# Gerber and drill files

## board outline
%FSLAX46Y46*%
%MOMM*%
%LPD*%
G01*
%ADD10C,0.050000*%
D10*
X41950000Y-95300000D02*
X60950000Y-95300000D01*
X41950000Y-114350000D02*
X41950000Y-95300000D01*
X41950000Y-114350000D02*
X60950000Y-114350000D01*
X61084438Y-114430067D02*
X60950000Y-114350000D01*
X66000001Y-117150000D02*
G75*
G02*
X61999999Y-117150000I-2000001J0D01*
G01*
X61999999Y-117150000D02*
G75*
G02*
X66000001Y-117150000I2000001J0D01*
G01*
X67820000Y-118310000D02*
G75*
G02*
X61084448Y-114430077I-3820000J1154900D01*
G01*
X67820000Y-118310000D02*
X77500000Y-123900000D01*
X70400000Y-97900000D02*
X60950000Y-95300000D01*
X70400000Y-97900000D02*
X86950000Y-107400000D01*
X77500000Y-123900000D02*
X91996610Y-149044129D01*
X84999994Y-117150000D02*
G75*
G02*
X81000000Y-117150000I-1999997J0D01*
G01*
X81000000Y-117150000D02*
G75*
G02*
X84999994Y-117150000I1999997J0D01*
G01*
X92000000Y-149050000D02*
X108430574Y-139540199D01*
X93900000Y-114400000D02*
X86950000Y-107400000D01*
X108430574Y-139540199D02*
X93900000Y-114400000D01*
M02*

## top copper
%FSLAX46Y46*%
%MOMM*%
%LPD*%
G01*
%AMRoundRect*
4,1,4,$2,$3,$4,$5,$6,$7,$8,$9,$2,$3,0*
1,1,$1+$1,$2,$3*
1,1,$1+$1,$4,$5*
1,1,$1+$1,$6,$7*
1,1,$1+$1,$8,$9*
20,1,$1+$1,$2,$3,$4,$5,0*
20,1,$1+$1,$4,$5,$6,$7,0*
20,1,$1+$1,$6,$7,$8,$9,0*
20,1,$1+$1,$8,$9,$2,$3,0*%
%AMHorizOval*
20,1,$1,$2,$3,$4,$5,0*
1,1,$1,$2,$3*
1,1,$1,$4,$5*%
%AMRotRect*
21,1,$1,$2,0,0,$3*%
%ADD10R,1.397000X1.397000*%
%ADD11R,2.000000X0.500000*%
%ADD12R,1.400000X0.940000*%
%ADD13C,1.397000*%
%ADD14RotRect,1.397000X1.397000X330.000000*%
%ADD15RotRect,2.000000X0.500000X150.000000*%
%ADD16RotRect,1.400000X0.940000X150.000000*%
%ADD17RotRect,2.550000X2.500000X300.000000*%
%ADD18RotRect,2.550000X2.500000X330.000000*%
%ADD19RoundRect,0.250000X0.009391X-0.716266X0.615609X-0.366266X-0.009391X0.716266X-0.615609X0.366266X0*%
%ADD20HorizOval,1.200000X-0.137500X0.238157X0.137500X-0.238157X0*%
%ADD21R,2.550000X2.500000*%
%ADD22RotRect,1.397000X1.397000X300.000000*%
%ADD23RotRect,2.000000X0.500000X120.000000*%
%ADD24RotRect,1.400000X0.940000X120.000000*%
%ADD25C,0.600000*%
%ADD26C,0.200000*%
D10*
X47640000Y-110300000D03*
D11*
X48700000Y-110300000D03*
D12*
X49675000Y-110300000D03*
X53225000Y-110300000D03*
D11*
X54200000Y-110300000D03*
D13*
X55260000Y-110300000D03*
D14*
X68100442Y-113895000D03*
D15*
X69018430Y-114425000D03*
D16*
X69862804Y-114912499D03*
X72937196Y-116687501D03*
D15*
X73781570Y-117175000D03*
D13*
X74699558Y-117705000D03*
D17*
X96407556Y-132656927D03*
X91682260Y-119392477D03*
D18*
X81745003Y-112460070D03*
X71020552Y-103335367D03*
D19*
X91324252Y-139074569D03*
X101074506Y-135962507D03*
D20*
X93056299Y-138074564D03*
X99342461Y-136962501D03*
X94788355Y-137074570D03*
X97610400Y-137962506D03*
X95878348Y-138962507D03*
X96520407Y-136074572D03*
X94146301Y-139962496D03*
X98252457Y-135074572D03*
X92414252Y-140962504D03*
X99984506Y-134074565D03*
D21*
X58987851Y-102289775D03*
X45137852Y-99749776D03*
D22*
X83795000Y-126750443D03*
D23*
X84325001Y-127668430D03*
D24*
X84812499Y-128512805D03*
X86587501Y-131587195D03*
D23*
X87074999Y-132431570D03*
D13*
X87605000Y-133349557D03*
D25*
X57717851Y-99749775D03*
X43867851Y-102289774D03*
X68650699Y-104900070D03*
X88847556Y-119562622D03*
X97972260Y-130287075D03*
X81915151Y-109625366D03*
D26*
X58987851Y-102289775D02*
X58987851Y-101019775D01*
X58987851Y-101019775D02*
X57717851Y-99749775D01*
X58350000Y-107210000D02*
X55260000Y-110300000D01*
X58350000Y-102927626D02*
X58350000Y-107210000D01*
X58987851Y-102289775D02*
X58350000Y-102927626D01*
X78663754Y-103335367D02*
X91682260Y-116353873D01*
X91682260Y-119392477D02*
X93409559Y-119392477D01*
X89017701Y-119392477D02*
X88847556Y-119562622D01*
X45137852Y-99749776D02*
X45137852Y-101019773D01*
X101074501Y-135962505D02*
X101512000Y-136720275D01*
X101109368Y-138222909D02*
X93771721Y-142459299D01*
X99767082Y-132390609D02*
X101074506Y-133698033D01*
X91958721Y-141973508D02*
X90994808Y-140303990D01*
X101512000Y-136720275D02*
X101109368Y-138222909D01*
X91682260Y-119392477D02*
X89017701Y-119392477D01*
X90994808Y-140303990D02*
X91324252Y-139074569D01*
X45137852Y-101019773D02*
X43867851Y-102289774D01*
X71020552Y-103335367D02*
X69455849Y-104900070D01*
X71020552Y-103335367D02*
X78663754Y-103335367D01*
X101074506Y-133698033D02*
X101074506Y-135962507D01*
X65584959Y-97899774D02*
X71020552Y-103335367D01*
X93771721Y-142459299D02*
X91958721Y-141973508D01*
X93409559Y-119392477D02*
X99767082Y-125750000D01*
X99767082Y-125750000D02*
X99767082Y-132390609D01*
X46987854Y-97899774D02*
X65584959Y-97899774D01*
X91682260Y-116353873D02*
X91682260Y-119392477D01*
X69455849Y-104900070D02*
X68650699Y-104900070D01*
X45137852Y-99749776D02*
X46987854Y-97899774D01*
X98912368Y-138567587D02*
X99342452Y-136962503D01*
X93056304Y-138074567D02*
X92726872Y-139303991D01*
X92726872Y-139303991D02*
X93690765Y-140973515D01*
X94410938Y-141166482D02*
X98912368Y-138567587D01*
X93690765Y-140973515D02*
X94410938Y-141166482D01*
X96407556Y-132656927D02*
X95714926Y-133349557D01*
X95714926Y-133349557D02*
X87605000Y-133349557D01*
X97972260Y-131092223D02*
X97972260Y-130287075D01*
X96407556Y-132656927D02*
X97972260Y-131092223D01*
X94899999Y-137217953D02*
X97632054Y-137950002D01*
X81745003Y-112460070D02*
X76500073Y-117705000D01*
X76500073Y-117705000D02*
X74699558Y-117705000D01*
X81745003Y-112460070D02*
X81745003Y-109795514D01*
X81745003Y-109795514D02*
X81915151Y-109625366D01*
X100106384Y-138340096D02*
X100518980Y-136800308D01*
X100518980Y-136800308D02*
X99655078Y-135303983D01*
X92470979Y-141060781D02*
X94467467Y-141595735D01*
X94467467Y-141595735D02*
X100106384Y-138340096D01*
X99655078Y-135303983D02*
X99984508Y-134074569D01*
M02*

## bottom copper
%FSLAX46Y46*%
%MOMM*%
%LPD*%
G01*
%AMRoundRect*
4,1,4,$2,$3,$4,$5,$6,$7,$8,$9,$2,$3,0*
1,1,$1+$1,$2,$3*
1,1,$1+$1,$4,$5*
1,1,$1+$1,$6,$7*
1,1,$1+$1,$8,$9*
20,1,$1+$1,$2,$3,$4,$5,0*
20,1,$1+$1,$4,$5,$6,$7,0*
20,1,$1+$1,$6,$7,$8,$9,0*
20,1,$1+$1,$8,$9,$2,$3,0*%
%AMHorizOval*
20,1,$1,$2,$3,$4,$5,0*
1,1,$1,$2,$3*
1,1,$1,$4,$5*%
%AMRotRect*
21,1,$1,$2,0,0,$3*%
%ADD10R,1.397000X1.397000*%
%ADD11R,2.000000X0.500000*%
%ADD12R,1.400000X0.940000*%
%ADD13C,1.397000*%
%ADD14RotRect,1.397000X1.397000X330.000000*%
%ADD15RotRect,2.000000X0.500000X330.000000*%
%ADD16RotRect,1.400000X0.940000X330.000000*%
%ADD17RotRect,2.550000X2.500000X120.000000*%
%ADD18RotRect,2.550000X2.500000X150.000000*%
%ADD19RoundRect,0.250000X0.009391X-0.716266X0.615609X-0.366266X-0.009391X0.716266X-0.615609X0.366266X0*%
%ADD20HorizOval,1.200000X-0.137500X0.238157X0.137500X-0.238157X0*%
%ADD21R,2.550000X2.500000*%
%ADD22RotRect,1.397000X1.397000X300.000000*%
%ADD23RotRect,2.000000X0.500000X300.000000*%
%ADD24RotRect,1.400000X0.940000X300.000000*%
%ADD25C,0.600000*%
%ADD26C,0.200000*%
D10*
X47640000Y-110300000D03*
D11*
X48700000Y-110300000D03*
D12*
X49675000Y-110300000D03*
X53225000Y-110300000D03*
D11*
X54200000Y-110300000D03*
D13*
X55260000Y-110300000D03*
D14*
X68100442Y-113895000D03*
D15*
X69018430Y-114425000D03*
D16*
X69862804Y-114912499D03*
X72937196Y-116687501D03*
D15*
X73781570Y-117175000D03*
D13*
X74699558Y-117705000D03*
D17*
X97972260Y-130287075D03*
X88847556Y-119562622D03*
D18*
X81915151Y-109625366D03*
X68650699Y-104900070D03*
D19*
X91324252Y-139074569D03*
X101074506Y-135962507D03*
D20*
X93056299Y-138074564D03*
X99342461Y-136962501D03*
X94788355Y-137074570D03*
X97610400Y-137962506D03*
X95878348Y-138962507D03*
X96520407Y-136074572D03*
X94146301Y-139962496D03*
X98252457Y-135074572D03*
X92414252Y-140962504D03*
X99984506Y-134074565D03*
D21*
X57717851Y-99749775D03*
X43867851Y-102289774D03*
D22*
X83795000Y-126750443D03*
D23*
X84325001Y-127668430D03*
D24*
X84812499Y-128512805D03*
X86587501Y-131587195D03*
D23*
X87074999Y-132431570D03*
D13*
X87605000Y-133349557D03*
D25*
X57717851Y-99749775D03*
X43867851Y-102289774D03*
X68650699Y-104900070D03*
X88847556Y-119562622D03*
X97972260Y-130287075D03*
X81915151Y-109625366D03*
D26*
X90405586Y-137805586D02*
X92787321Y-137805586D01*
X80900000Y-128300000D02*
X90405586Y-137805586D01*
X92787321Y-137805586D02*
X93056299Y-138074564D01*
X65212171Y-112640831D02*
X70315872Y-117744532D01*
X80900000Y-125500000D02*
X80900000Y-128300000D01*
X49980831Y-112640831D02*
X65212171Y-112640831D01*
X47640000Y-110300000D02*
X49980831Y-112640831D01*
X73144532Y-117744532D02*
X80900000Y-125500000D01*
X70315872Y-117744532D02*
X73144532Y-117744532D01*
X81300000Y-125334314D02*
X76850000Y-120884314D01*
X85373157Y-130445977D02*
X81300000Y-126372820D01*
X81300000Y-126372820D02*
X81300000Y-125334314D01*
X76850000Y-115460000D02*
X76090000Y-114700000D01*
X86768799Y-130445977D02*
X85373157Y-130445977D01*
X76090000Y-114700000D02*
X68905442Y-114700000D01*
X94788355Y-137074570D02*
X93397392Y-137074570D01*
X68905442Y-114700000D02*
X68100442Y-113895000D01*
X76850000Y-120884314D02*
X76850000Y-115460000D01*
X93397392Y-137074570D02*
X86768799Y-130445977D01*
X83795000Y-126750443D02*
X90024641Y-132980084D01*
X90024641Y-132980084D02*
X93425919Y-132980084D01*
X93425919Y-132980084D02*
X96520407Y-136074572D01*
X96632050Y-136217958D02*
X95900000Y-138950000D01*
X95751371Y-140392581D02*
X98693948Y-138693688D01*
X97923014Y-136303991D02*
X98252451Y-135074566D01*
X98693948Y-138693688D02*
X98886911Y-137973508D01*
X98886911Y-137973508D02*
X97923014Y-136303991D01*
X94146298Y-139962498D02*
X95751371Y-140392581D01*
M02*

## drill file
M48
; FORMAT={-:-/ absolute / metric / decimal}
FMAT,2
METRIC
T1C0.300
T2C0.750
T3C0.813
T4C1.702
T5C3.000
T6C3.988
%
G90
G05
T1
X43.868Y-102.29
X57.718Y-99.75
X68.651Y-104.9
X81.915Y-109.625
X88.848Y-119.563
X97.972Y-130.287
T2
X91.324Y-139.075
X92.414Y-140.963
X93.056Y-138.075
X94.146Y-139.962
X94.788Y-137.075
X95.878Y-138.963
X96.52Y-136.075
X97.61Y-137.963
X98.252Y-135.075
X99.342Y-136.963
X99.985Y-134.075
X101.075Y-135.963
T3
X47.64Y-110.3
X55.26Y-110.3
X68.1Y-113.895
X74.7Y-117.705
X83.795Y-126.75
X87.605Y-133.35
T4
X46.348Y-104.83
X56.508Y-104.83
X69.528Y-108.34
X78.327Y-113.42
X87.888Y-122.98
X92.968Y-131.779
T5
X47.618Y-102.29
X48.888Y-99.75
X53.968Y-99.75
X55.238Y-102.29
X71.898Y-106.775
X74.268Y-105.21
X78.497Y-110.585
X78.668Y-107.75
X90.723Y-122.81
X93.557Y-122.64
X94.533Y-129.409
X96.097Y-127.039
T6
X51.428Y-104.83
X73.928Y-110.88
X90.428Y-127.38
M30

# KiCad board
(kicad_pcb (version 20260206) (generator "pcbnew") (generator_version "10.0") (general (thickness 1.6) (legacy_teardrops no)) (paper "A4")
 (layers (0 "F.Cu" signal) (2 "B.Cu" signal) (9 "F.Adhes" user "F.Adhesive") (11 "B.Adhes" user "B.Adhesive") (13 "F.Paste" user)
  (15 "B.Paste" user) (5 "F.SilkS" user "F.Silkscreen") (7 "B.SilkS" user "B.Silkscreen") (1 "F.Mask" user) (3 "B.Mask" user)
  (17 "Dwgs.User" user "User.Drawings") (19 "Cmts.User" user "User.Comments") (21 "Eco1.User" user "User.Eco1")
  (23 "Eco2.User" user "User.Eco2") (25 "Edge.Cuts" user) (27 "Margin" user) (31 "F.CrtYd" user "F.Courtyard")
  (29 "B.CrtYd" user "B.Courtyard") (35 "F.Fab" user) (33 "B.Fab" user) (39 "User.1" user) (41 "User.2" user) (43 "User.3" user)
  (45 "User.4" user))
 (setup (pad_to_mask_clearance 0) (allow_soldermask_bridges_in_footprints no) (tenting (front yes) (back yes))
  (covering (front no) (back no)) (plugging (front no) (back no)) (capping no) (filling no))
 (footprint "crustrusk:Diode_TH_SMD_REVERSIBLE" (layer "F.Cu") (at 51.45 110.3)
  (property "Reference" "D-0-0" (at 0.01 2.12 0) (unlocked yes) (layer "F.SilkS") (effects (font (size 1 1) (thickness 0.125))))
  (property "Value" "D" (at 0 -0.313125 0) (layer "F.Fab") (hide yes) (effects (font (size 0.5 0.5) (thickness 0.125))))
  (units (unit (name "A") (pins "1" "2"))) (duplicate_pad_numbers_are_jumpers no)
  (pad "1" thru_hole rect (at -3.81 0) (size 1.397 1.397) (drill 0.8128) (layers "*.Cu" "*.Mask") (remove_unused_layers no) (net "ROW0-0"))
  (pad "1" smd rect (at -2.75 0 180) (size 2 0.5) (layers "F.Cu") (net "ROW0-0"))
  (pad "1" smd rect (at -2.75 0) (size 2 0.5) (layers "B.Cu") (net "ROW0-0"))
  (pad "1" smd rect (at -1.775 0 180) (size 1.4 0.94) (layers "F.Cu" "F.Mask" "F.Paste") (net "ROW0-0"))
  (pad "1" smd rect (at -1.775 0) (size 1.4 0.94) (layers "B.Cu" "B.Mask" "B.Paste") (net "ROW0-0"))
  (pad "2" smd rect (at 1.775 0 180) (size 1.4 0.94) (layers "F.Cu" "F.Mask" "F.Paste") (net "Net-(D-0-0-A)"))
  (pad "2" smd rect (at 1.775 0) (size 1.4 0.94) (layers "B.Cu" "B.Mask" "B.Paste") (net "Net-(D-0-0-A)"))
  (pad "2" smd rect (at 2.75 0 180) (size 2 0.5) (layers "F.Cu") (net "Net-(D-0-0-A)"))
  (pad "2" smd rect (at 2.75 0) (size 2 0.5) (layers "B.Cu") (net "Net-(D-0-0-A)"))
  (pad "2" thru_hole circle (at 3.81 0) (size 1.397 1.397) (drill 0.8128) (layers "*.Cu" "*.Mask") (remove_unused_layers no)
   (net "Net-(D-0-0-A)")))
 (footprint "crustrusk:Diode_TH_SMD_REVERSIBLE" (layer "F.Cu") (at 71.4 115.8 -30)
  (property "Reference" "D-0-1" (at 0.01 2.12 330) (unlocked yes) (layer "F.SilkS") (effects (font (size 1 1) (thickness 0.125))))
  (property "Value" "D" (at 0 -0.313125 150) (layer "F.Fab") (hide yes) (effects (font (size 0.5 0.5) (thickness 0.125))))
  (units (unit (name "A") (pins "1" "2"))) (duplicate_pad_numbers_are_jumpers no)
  (pad "1" thru_hole rect (at -3.810001 0.000001 330) (size 1.397 1.397) (drill 0.8128) (layers "*.Cu" "*.Mask") (remove_unused_layers no)
   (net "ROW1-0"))
  (pad "1" smd rect (at -2.75 0 150) (size 2 0.5) (layers "F.Cu") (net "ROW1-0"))
  (pad "1" smd rect (at -2.75 0 330) (size 2 0.5) (layers "B.Cu") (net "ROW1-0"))
  (pad "1" smd rect (at -1.775001 0 150) (size 1.4 0.94) (layers "F.Cu" "F.Mask" "F.Paste") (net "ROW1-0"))
  (pad "1" smd rect (at -1.775001 0 330) (size 1.4 0.94) (layers "B.Cu" "B.Mask" "B.Paste") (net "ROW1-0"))
  (pad "2" smd rect (at 1.775001 0 150) (size 1.4 0.94) (layers "F.Cu" "F.Mask" "F.Paste") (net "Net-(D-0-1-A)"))
  (pad "2" smd rect (at 1.775001 0 330) (size 1.4 0.94) (layers "B.Cu" "B.Mask" "B.Paste") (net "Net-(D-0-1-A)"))
  (pad "2" smd rect (at 2.75 0 150) (size 2 0.5) (layers "F.Cu") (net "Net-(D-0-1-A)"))
  (pad "2" smd rect (at 2.75 0 330) (size 2 0.5) (layers "B.Cu") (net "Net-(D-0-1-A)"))
  (pad "2" thru_hole circle (at 3.810001 -0.000001 330) (size 1.397 1.397) (drill 0.8128) (layers "*.Cu" "*.Mask") (remove_unused_layers no)
   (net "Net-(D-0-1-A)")))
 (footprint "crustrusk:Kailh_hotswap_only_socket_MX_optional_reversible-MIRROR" (layer "F.Cu") (at 90.427851 127.379775 -60)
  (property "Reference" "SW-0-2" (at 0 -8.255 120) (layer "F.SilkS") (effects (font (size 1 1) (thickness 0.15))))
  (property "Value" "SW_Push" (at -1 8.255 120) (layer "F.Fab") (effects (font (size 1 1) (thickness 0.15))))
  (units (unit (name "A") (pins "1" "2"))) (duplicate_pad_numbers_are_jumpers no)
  (pad "" np_thru_hole circle (at -5.08 0 300) (size 1.7018 1.7018) (drill 1.7018) (layers "*.Cu" "*.Mask"))
  (pad "" np_thru_hole circle (at -3.81 -2.540001 120) (size 3 3) (drill 3) (layers "*.Cu" "*.Mask"))
  (pad "" np_thru_hole circle (at -2.540001 -5.079998 300) (size 3 3) (drill 3) (layers "*.Cu" "*.Mask"))
  (pad "" np_thru_hole circle (at 0 0 300) (size 3.9878 3.9878) (drill 3.9878) (layers "*.Cu" "*.Mask"))
  (pad "" np_thru_hole circle (at 2.540002 -5.080001 120) (size 3 3) (drill 3) (layers "*.Cu" "*.Mask"))
  (pad "" np_thru_hole circle (at 3.81 -2.54 300) (size 3 3) (drill 3) (layers "*.Cu" "*.Mask"))
  (pad "" np_thru_hole circle (at 5.08 0 300) (size 1.7018 1.7018) (drill 1.7018) (layers "*.Cu" "*.Mask"))
  (pad "1" smd rect (at 6.29 -5.08 120) (size 2.55 2.5) (layers "B.Cu" "B.Mask" "B.Paste") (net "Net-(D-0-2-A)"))
  (pad "1" smd rect (at 7.56 -2.54 300) (size 2.55 2.5) (layers "F.Cu" "F.Mask" "F.Paste") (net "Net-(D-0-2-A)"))
  (pad "2" smd rect (at -7.560001 -2.540001 120) (size 2.55 2.5) (layers "B.Cu" "B.Mask" "B.Paste") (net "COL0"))
  (pad "2" smd rect (at -6.289998 -5.079999 300) (size 2.55 2.5) (layers "F.Cu" "F.Mask" "F.Paste") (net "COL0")))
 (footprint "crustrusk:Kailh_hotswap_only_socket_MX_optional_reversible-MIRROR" (layer "F.Cu") (at 73.927851 110.879775 -30)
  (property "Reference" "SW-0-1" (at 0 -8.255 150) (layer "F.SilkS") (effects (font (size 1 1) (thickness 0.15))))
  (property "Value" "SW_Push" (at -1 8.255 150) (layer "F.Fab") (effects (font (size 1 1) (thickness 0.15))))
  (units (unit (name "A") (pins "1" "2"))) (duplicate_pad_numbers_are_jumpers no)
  (pad "" np_thru_hole circle (at -5.08 0 330) (size 1.7018 1.7018) (drill 1.7018) (layers "*.Cu" "*.Mask"))
  (pad "" np_thru_hole circle (at -3.81 -2.54 150) (size 3 3) (drill 3) (layers "*.Cu" "*.Mask"))
  (pad "" np_thru_hole circle (at -2.54 -5.079997 330) (size 3 3) (drill 3) (layers "*.Cu" "*.Mask"))
  (pad "" np_thru_hole circle (at 0 0 330) (size 3.9878 3.9878) (drill 3.9878) (layers "*.Cu" "*.Mask"))
  (pad "" np_thru_hole circle (at 2.540002 -5.080001 150) (size 3 3) (drill 3) (layers "*.Cu" "*.Mask"))
  (pad "" np_thru_hole circle (at 3.81 -2.540001 330) (size 3 3) (drill 3) (layers "*.Cu" "*.Mask"))
  (pad "" np_thru_hole circle (at 5.08 0 330) (size 1.7018 1.7018) (drill 1.7018) (layers "*.Cu" "*.Mask"))
  (pad "1" smd rect (at 6.29 -5.08 150) (size 2.55 2.5) (layers "B.Cu" "B.Mask" "B.Paste") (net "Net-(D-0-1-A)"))
  (pad "1" smd rect (at 7.56 -2.54 330) (size 2.55 2.5) (layers "F.Cu" "F.Mask" "F.Paste") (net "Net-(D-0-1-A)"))
  (pad "2" smd rect (at -7.56 -2.54 150) (size 2.55 2.5) (layers "B.Cu" "B.Mask" "B.Paste") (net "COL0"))
  (pad "2" smd rect (at -6.289999 -5.079999 330) (size 2.55 2.5) (layers "F.Cu" "F.Mask" "F.Paste") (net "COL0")))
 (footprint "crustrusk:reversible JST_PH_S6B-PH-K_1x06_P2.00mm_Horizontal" (layer "F.Cu") (at 91.324252 139.074569 30)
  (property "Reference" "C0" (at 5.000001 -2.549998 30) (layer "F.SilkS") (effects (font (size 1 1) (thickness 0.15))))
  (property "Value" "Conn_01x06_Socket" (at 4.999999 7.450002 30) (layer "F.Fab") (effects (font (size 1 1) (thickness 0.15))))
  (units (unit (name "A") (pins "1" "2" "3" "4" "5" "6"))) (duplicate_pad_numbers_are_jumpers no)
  (pad "1" thru_hole roundrect (at 0 0 30) (size 1.2 1.75) (drill 0.75) (layers "*.Cu" "*.Mask") (remove_unused_layers no)
   (roundrect_rratio 0.208333) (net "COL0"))
  (pad "1" thru_hole roundrect (at 9.999999 2.180002 30) (size 1.2 1.75) (drill 0.75) (layers "*.Cu" "*.Mask") (remove_unused_layers no)
   (roundrect_rratio 0.208333) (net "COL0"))
  (pad "2" thru_hole oval (at 1.999999 -0.000006 30) (size 1.2 1.75) (drill 0.75) (layers "*.Cu" "*.Mask") (remove_unused_layers no)
   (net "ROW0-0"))
  (pad "2" thru_hole oval (at 8.000007 2.18 30) (size 1.2 1.75) (drill 0.75) (layers "*.Cu" "*.Mask") (remove_unused_layers no)
   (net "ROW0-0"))
  (pad "3" thru_hole oval (at 4.000001 0.000002 30) (size 1.2 1.75) (drill 0.75) (layers "*.Cu" "*.Mask") (remove_unused_layers no)
   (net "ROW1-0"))
  (pad "3" thru_hole oval (at 5.999995 2.179999 30) (size 1.2 1.75) (drill 0.75) (layers "*.Cu" "*.Mask") (remove_unused_layers no)
   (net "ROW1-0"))
  (pad "4" thru_hole oval (at 3.999994 2.179999 30) (size 1.2 1.75) (drill 0.75) (layers "*.Cu" "*.Mask") (remove_unused_layers no)
   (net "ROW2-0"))
  (pad "4" thru_hole oval (at 6.000001 0.000004 30) (size 1.2 1.75) (drill 0.75) (layers "*.Cu" "*.Mask") (remove_unused_layers no)
   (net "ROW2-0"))
  (pad "5" thru_hole oval (at 2.000003 2.179992 30) (size 1.2 1.75) (drill 0.75) (layers "*.Cu" "*.Mask") (remove_unused_layers no)
   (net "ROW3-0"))
  (pad "5" thru_hole oval (at 8 0.000003 30) (size 1.2 1.75) (drill 0.75) (layers "*.Cu" "*.Mask") (remove_unused_layers no) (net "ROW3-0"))
  (pad "6" thru_hole oval (at 0 2.18 30) (size 1.2 1.75) (drill 0.75) (layers "*.Cu" "*.Mask") (remove_unused_layers no) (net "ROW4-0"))
  (pad "6" thru_hole oval (at 10.000002 -0.000004 30) (size 1.2 1.75) (drill 0.75) (layers "*.Cu" "*.Mask") (remove_unused_layers no)
   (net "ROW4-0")))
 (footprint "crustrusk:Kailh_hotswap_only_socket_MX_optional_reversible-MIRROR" (layer "F.Cu") (at 51.427851 104.829775)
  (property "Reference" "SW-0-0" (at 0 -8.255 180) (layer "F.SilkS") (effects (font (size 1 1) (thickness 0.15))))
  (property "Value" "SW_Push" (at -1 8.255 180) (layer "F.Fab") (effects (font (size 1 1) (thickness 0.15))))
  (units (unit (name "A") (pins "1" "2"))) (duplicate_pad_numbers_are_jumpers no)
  (pad "" np_thru_hole circle (at -5.08 0) (size 1.7018 1.7018) (drill 1.7018) (layers "*.Cu" "*.Mask"))
  (pad "" np_thru_hole circle (at -3.81 -2.54 180) (size 3 3) (drill 3) (layers "*.Cu" "*.Mask"))
  (pad "" np_thru_hole circle (at -2.54 -5.079998) (size 3 3) (drill 3) (layers "*.Cu" "*.Mask"))
  (pad "" np_thru_hole circle (at 0 0) (size 3.9878 3.9878) (drill 3.9878) (layers "*.Cu" "*.Mask"))
  (pad "" np_thru_hole circle (at 2.540002 -5.080001 180) (size 3 3) (drill 3) (layers "*.Cu" "*.Mask"))
  (pad "" np_thru_hole circle (at 3.81 -2.54) (size 3 3) (drill 3) (layers "*.Cu" "*.Mask"))
  (pad "" np_thru_hole circle (at 5.08 0) (size 1.7018 1.7018) (drill 1.7018) (layers "*.Cu" "*.Mask"))
  (pad "1" smd rect (at 6.29 -5.08 180) (size 2.55 2.5) (layers "B.Cu" "B.Mask" "B.Paste") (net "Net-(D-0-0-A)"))
  (pad "1" smd rect (at 7.56 -2.54) (size 2.55 2.5) (layers "F.Cu" "F.Mask" "F.Paste") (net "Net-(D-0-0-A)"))
  (pad "2" smd rect (at -7.56 -2.540001 180) (size 2.55 2.5) (layers "B.Cu" "B.Mask" "B.Paste") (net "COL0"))
  (pad "2" smd rect (at -6.289999 -5.079999) (size 2.55 2.5) (layers "F.Cu" "F.Mask" "F.Paste") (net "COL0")))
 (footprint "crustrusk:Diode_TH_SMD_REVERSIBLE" (layer "F.Cu") (at 85.7 130.05 -60)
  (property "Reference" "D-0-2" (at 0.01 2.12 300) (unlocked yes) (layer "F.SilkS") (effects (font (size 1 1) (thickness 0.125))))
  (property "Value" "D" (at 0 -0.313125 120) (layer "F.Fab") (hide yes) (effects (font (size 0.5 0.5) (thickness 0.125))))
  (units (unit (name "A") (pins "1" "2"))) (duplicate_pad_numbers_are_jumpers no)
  (pad "1" thru_hole rect (at -3.81 0 300) (size 1.397 1.397) (drill 0.8128) (layers "*.Cu" "*.Mask") (remove_unused_layers no)
   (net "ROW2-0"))
  (pad "1" smd rect (at -2.75 -0.000001 120) (size 2 0.5) (layers "F.Cu") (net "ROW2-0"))
  (pad "1" smd rect (at -2.75 -0.000001 300) (size 2 0.5) (layers "B.Cu") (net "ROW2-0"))
  (pad "1" smd rect (at -1.775 0.000001 120) (size 1.4 0.94) (layers "F.Cu" "F.Mask" "F.Paste") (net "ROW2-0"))
  (pad "1" smd rect (at -1.775 0.000001 300) (size 1.4 0.94) (layers "B.Cu" "B.Mask" "B.Paste") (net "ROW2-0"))
  (pad "2" smd rect (at 1.775 -0.000001 120) (size 1.4 0.94) (layers "F.Cu" "F.Mask" "F.Paste") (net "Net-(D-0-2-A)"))
  (pad "2" smd rect (at 1.775 -0.000001 300) (size 1.4 0.94) (layers "B.Cu" "B.Mask" "B.Paste") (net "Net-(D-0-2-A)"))
  (pad "2" smd rect (at 2.75 0.000001 120) (size 2 0.5) (layers "F.Cu") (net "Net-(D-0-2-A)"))
  (pad "2" smd rect (at 2.75 0.000001 300) (size 2 0.5) (layers "B.Cu") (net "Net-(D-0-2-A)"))
  (pad "2" thru_hole circle (at 3.81 0 300) (size 1.397 1.397) (drill 0.8128) (layers "*.Cu" "*.Mask") (remove_unused_layers no)
   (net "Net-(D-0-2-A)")))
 (gr_line (start 41.95 95.3) (end 60.95 95.3) (stroke (width 0.05) (type default)) (layer "Edge.Cuts"))
 (gr_line (start 41.95 114.35) (end 41.95 95.3) (stroke (width 0.05) (type default)) (layer "Edge.Cuts"))
 (gr_line (start 41.95 114.35) (end 60.95 114.35) (stroke (width 0.05) (type default)) (layer "Edge.Cuts"))
 (gr_line (start 61.084438 114.430067) (end 60.95 114.35) (stroke (width 0.05) (type default)) (layer "Edge.Cuts"))
 (gr_circle (center 64 117.15) (end 61.999999 117.15) (stroke (width 0.05) (type default)) (fill no) (layer "Edge.Cuts"))
 (gr_arc (start 67.82 118.31) (mid 62.008023 120.613157) (end 61.084438 114.430067) (stroke (width 0.05) (type default)) (layer "Edge.Cuts"))
 (gr_line (start 67.82 118.31) (end 77.5 123.9) (stroke (width 0.05) (type default)) (layer "Edge.Cuts"))
 (gr_line (start 70.4 97.9) (end 60.95 95.3) (stroke (width 0.05) (type default)) (layer "Edge.Cuts"))
 (gr_line (start 70.4 97.9) (end 86.95 107.4) (stroke (width 0.05) (type default)) (layer "Edge.Cuts"))
 (gr_line (start 77.5 123.9) (end 91.99661 149.044129) (stroke (width 0.05) (type default)) (layer "Edge.Cuts"))
 (gr_circle (center 82.999997 117.15) (end 81 117.15) (stroke (width 0.05) (type default)) (fill no) (layer "Edge.Cuts"))
 (gr_line (start 92 149.05) (end 108.430574 139.540199) (stroke (width 0.05) (type default)) (layer "Edge.Cuts"))
 (gr_line (start 93.9 114.4) (end 86.95 107.4) (stroke (width 0.05) (type default)) (layer "Edge.Cuts"))
 (gr_line (start 108.430574 139.540199) (end 93.9 114.4) (stroke (width 0.05) (type default)) (layer "Edge.Cuts"))
 (segment (start 58.987851 102.289775) (end 58.987851 101.019775) (width 0.2) (layer "F.Cu") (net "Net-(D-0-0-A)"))
 (segment (start 58.987851 101.019775) (end 57.717851 99.749775) (width 0.2) (layer "F.Cu") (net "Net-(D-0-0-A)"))
 (segment (start 58.35 107.21) (end 55.26 110.3) (width 0.2) (layer "F.Cu") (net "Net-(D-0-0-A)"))
 (segment (start 58.35 102.927626) (end 58.35 107.21) (width 0.2) (layer "F.Cu") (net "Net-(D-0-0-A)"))
 (segment (start 58.987851 102.289775) (end 58.35 102.927626) (width 0.2) (layer "F.Cu") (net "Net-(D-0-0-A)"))
 (via (at 57.717851 99.749775) (size 0.6) (drill 0.3) (layers "F.Cu" "B.Cu") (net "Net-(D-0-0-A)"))
 (segment (start 78.663754 103.335367) (end 91.68226 116.353873) (width 0.2) (layer "F.Cu") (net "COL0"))
 (segment (start 91.68226 119.392477) (end 93.409559 119.392477) (width 0.2) (layer "F.Cu") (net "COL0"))
 (segment (start 89.017701 119.392477) (end 88.847556 119.562622) (width 0.2) (layer "F.Cu") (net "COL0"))
 (segment (start 45.137852 99.749776) (end 45.137852 101.019773) (width 0.2) (layer "F.Cu") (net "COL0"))
 (segment (start 101.074501 135.962505) (end 101.512 136.720275) (width 0.2) (layer "F.Cu") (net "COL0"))
 (segment (start 101.109368 138.222909) (end 93.771721 142.459299) (width 0.2) (layer "F.Cu") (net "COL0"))
 (segment (start 99.767082 132.390609) (end 101.074506 133.698033) (width 0.2) (layer "F.Cu") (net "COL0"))
 (segment (start 91.958721 141.973508) (end 90.994808 140.30399) (width 0.2) (layer "F.Cu") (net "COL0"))
 (segment (start 101.512 136.720275) (end 101.109368 138.222909) (width 0.2) (layer "F.Cu") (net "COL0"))
 (segment (start 91.68226 119.392477) (end 89.017701 119.392477) (width 0.2) (layer "F.Cu") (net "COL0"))
 (segment (start 90.994808 140.30399) (end 91.324252 139.074569) (width 0.2) (layer "F.Cu") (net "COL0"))
 (segment (start 45.137852 101.019773) (end 43.867851 102.289774) (width 0.2) (layer "F.Cu") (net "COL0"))
 (segment (start 71.020552 103.335367) (end 69.455849 104.90007) (width 0.2) (layer "F.Cu") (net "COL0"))
 (segment (start 71.020552 103.335367) (end 78.663754 103.335367) (width 0.2) (layer "F.Cu") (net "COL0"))
 (segment (start 101.074506 133.698033) (end 101.074506 135.962507) (width 0.2) (layer "F.Cu") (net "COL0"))
 (segment (start 65.584959 97.899774) (end 71.020552 103.335367) (width 0.2) (layer "F.Cu") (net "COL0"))
 (segment (start 93.771721 142.459299) (end 91.958721 141.973508) (width 0.2) (layer "F.Cu") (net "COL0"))
 (segment (start 93.409559 119.392477) (end 99.767082 125.75) (width 0.2) (layer "F.Cu") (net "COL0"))
 (segment (start 99.767082 125.75) (end 99.767082 132.390609) (width 0.2) (layer "F.Cu") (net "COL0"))
 (segment (start 46.987854 97.899774) (end 65.584959 97.899774) (width 0.2) (layer "F.Cu") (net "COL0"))
 (segment (start 91.68226 116.353873) (end 91.68226 119.392477) (width 0.2) (layer "F.Cu") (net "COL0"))
 (segment (start 69.455849 104.90007) (end 68.650699 104.90007) (width 0.2) (layer "F.Cu") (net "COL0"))
 (segment (start 45.137852 99.749776) (end 46.987854 97.899774) (width 0.2) (layer "F.Cu") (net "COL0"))
 (via (at 43.867851 102.289774) (size 0.6) (drill 0.3) (layers "F.Cu" "B.Cu") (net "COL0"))
 (via (at 68.650699 104.90007) (size 0.6) (drill 0.3) (layers "F.Cu" "B.Cu") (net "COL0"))
 (via (at 88.847556 119.562622) (size 0.6) (drill 0.3) (layers "F.Cu" "B.Cu") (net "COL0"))
 (segment (start 98.912368 138.567587) (end 99.342452 136.962503) (width 0.2) (layer "F.Cu") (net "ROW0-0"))
 (segment (start 93.056304 138.074567) (end 92.726872 139.303991) (width 0.2) (layer "F.Cu") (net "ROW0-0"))
 (segment (start 92.726872 139.303991) (end 93.690765 140.973515) (width 0.2) (layer "F.Cu") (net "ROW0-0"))
 (segment (start 94.410938 141.166482) (end 98.912368 138.567587) (width 0.2) (layer "F.Cu") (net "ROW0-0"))
 (segment (start 93.690765 140.973515) (end 94.410938 141.166482) (width 0.2) (layer "F.Cu") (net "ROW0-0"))
 (segment (start 90.405586 137.805586) (end 92.787321 137.805586) (width 0.2) (layer "B.Cu") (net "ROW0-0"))
 (segment (start 80.9 128.3) (end 90.405586 137.805586) (width 0.2) (layer "B.Cu") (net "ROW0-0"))
 (segment (start 92.787321 137.805586) (end 93.056299 138.074564) (width 0.2) (layer "B.Cu") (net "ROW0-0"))
 (segment (start 65.212171 112.640831) (end 70.315872 117.744532) (width 0.2) (layer "B.Cu") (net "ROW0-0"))
 (segment (start 80.9 125.5) (end 80.9 128.3) (width 0.2) (layer "B.Cu") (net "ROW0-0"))
 (segment (start 49.980831 112.640831) (end 65.212171 112.640831) (width 0.2) (layer "B.Cu") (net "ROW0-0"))
 (segment (start 47.64 110.3) (end 49.980831 112.640831) (width 0.2) (layer "B.Cu") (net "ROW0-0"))
 (segment (start 73.144532 117.744532) (end 80.9 125.5) (width 0.2) (layer "B.Cu") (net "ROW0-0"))
 (segment (start 70.315872 117.744532) (end 73.144532 117.744532) (width 0.2) (layer "B.Cu") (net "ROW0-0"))
 (segment (start 96.407556 132.656927) (end 95.714926 133.349557) (width 0.2) (layer "F.Cu") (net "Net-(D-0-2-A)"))
 (segment (start 95.714926 133.349557) (end 87.605 133.349557) (width 0.2) (layer "F.Cu") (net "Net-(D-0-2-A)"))
 (segment (start 97.97226 131.092223) (end 97.97226 130.287075) (width 0.2) (layer "F.Cu") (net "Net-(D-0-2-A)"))
 (segment (start 96.407556 132.656927) (end 97.97226 131.092223) (width 0.2) (layer "F.Cu") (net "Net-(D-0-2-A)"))
 (via (at 97.97226 130.287075) (size 0.6) (drill 0.3) (layers "F.Cu" "B.Cu") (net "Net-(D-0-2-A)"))
 (segment (start 94.899999 137.217953) (end 97.632054 137.950002) (width 0.2) (layer "F.Cu") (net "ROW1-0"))
 (segment (start 81.3 125.334314) (end 76.85 120.884314) (width 0.2) (layer "B.Cu") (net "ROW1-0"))
 (segment (start 85.373157 130.445977) (end 81.3 126.37282) (width 0.2) (layer "B.Cu") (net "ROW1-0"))
 (segment (start 81.3 126.37282) (end 81.3 125.334314) (width 0.2) (layer "B.Cu") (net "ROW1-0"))
 (segment (start 76.85 115.46) (end 76.09 114.7) (width 0.2) (layer "B.Cu") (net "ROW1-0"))
 (segment (start 86.768799 130.445977) (end 85.373157 130.445977) (width 0.2) (layer "B.Cu") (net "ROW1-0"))
 (segment (start 76.09 114.7) (end 68.905442 114.7) (width 0.2) (layer "B.Cu") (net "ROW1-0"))
 (segment (start 94.788355 137.07457) (end 93.397392 137.07457) (width 0.2) (layer "B.Cu") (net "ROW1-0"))
 (segment (start 68.905442 114.7) (end 68.100442 113.895) (width 0.2) (layer "B.Cu") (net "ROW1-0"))
 (segment (start 76.85 120.884314) (end 76.85 115.46) (width 0.2) (layer "B.Cu") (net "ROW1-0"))
 (segment (start 93.397392 137.07457) (end 86.768799 130.445977) (width 0.2) (layer "B.Cu") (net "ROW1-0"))
 (segment (start 81.745003 112.46007) (end 76.500073 117.705) (width 0.2) (layer "F.Cu") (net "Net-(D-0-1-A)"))
 (segment (start 76.500073 117.705) (end 74.699558 117.705) (width 0.2) (layer "F.Cu") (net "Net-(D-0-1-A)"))
 (segment (start 81.745003 112.46007) (end 81.745003 109.795514) (width 0.2) (layer "F.Cu") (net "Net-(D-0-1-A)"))
 (segment (start 81.745003 109.795514) (end 81.915151 109.625366) (width 0.2) (layer "F.Cu") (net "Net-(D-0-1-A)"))
 (via (at 81.915151 109.625366) (size 0.6) (drill 0.3) (layers "F.Cu" "B.Cu") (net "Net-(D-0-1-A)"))
 (segment (start 83.795 126.750443) (end 90.024641 132.980084) (width 0.2) (layer "B.Cu") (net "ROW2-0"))
 (segment (start 90.024641 132.980084) (end 93.425919 132.980084) (width 0.2) (layer "B.Cu") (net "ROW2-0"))
 (segment (start 93.425919 132.980084) (end 96.520407 136.074572) (width 0.2) (layer "B.Cu") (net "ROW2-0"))
 (segment (start 96.63205 136.217958) (end 95.9 138.95) (width 0.2) (layer "B.Cu") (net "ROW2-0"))
 (segment (start 95.751371 140.392581) (end 98.693948 138.693688) (width 0.2) (layer "B.Cu") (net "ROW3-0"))
 (segment (start 97.923014 136.303991) (end 98.252451 135.074566) (width 0.2) (layer "B.Cu") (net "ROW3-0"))
 (segment (start 98.693948 138.693688) (end 98.886911 137.973508) (width 0.2) (layer "B.Cu") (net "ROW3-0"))
 (segment (start 98.886911 137.973508) (end 97.923014 136.303991) (width 0.2) (layer "B.Cu") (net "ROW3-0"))
 (segment (start 94.146298 139.962498) (end 95.751371 140.392581) (width 0.2) (layer "B.Cu") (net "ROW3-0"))
 (segment (start 100.106384 138.340096) (end 100.51898 136.800308) (width 0.2) (layer "F.Cu") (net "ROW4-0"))
 (segment (start 100.51898 136.800308) (end 99.655078 135.303983) (width 0.2) (layer "F.Cu") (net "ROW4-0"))
 (segment (start 92.470979 141.060781) (end 94.467467 141.595735) (width 0.2) (layer "F.Cu") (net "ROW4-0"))
 (segment (start 94.467467 141.595735) (end 100.106384 138.340096) (width 0.2) (layer "F.Cu") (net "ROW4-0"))
 (segment (start 99.655078 135.303983) (end 99.984508 134.074569) (width 0.2) (layer "F.Cu") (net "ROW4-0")))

